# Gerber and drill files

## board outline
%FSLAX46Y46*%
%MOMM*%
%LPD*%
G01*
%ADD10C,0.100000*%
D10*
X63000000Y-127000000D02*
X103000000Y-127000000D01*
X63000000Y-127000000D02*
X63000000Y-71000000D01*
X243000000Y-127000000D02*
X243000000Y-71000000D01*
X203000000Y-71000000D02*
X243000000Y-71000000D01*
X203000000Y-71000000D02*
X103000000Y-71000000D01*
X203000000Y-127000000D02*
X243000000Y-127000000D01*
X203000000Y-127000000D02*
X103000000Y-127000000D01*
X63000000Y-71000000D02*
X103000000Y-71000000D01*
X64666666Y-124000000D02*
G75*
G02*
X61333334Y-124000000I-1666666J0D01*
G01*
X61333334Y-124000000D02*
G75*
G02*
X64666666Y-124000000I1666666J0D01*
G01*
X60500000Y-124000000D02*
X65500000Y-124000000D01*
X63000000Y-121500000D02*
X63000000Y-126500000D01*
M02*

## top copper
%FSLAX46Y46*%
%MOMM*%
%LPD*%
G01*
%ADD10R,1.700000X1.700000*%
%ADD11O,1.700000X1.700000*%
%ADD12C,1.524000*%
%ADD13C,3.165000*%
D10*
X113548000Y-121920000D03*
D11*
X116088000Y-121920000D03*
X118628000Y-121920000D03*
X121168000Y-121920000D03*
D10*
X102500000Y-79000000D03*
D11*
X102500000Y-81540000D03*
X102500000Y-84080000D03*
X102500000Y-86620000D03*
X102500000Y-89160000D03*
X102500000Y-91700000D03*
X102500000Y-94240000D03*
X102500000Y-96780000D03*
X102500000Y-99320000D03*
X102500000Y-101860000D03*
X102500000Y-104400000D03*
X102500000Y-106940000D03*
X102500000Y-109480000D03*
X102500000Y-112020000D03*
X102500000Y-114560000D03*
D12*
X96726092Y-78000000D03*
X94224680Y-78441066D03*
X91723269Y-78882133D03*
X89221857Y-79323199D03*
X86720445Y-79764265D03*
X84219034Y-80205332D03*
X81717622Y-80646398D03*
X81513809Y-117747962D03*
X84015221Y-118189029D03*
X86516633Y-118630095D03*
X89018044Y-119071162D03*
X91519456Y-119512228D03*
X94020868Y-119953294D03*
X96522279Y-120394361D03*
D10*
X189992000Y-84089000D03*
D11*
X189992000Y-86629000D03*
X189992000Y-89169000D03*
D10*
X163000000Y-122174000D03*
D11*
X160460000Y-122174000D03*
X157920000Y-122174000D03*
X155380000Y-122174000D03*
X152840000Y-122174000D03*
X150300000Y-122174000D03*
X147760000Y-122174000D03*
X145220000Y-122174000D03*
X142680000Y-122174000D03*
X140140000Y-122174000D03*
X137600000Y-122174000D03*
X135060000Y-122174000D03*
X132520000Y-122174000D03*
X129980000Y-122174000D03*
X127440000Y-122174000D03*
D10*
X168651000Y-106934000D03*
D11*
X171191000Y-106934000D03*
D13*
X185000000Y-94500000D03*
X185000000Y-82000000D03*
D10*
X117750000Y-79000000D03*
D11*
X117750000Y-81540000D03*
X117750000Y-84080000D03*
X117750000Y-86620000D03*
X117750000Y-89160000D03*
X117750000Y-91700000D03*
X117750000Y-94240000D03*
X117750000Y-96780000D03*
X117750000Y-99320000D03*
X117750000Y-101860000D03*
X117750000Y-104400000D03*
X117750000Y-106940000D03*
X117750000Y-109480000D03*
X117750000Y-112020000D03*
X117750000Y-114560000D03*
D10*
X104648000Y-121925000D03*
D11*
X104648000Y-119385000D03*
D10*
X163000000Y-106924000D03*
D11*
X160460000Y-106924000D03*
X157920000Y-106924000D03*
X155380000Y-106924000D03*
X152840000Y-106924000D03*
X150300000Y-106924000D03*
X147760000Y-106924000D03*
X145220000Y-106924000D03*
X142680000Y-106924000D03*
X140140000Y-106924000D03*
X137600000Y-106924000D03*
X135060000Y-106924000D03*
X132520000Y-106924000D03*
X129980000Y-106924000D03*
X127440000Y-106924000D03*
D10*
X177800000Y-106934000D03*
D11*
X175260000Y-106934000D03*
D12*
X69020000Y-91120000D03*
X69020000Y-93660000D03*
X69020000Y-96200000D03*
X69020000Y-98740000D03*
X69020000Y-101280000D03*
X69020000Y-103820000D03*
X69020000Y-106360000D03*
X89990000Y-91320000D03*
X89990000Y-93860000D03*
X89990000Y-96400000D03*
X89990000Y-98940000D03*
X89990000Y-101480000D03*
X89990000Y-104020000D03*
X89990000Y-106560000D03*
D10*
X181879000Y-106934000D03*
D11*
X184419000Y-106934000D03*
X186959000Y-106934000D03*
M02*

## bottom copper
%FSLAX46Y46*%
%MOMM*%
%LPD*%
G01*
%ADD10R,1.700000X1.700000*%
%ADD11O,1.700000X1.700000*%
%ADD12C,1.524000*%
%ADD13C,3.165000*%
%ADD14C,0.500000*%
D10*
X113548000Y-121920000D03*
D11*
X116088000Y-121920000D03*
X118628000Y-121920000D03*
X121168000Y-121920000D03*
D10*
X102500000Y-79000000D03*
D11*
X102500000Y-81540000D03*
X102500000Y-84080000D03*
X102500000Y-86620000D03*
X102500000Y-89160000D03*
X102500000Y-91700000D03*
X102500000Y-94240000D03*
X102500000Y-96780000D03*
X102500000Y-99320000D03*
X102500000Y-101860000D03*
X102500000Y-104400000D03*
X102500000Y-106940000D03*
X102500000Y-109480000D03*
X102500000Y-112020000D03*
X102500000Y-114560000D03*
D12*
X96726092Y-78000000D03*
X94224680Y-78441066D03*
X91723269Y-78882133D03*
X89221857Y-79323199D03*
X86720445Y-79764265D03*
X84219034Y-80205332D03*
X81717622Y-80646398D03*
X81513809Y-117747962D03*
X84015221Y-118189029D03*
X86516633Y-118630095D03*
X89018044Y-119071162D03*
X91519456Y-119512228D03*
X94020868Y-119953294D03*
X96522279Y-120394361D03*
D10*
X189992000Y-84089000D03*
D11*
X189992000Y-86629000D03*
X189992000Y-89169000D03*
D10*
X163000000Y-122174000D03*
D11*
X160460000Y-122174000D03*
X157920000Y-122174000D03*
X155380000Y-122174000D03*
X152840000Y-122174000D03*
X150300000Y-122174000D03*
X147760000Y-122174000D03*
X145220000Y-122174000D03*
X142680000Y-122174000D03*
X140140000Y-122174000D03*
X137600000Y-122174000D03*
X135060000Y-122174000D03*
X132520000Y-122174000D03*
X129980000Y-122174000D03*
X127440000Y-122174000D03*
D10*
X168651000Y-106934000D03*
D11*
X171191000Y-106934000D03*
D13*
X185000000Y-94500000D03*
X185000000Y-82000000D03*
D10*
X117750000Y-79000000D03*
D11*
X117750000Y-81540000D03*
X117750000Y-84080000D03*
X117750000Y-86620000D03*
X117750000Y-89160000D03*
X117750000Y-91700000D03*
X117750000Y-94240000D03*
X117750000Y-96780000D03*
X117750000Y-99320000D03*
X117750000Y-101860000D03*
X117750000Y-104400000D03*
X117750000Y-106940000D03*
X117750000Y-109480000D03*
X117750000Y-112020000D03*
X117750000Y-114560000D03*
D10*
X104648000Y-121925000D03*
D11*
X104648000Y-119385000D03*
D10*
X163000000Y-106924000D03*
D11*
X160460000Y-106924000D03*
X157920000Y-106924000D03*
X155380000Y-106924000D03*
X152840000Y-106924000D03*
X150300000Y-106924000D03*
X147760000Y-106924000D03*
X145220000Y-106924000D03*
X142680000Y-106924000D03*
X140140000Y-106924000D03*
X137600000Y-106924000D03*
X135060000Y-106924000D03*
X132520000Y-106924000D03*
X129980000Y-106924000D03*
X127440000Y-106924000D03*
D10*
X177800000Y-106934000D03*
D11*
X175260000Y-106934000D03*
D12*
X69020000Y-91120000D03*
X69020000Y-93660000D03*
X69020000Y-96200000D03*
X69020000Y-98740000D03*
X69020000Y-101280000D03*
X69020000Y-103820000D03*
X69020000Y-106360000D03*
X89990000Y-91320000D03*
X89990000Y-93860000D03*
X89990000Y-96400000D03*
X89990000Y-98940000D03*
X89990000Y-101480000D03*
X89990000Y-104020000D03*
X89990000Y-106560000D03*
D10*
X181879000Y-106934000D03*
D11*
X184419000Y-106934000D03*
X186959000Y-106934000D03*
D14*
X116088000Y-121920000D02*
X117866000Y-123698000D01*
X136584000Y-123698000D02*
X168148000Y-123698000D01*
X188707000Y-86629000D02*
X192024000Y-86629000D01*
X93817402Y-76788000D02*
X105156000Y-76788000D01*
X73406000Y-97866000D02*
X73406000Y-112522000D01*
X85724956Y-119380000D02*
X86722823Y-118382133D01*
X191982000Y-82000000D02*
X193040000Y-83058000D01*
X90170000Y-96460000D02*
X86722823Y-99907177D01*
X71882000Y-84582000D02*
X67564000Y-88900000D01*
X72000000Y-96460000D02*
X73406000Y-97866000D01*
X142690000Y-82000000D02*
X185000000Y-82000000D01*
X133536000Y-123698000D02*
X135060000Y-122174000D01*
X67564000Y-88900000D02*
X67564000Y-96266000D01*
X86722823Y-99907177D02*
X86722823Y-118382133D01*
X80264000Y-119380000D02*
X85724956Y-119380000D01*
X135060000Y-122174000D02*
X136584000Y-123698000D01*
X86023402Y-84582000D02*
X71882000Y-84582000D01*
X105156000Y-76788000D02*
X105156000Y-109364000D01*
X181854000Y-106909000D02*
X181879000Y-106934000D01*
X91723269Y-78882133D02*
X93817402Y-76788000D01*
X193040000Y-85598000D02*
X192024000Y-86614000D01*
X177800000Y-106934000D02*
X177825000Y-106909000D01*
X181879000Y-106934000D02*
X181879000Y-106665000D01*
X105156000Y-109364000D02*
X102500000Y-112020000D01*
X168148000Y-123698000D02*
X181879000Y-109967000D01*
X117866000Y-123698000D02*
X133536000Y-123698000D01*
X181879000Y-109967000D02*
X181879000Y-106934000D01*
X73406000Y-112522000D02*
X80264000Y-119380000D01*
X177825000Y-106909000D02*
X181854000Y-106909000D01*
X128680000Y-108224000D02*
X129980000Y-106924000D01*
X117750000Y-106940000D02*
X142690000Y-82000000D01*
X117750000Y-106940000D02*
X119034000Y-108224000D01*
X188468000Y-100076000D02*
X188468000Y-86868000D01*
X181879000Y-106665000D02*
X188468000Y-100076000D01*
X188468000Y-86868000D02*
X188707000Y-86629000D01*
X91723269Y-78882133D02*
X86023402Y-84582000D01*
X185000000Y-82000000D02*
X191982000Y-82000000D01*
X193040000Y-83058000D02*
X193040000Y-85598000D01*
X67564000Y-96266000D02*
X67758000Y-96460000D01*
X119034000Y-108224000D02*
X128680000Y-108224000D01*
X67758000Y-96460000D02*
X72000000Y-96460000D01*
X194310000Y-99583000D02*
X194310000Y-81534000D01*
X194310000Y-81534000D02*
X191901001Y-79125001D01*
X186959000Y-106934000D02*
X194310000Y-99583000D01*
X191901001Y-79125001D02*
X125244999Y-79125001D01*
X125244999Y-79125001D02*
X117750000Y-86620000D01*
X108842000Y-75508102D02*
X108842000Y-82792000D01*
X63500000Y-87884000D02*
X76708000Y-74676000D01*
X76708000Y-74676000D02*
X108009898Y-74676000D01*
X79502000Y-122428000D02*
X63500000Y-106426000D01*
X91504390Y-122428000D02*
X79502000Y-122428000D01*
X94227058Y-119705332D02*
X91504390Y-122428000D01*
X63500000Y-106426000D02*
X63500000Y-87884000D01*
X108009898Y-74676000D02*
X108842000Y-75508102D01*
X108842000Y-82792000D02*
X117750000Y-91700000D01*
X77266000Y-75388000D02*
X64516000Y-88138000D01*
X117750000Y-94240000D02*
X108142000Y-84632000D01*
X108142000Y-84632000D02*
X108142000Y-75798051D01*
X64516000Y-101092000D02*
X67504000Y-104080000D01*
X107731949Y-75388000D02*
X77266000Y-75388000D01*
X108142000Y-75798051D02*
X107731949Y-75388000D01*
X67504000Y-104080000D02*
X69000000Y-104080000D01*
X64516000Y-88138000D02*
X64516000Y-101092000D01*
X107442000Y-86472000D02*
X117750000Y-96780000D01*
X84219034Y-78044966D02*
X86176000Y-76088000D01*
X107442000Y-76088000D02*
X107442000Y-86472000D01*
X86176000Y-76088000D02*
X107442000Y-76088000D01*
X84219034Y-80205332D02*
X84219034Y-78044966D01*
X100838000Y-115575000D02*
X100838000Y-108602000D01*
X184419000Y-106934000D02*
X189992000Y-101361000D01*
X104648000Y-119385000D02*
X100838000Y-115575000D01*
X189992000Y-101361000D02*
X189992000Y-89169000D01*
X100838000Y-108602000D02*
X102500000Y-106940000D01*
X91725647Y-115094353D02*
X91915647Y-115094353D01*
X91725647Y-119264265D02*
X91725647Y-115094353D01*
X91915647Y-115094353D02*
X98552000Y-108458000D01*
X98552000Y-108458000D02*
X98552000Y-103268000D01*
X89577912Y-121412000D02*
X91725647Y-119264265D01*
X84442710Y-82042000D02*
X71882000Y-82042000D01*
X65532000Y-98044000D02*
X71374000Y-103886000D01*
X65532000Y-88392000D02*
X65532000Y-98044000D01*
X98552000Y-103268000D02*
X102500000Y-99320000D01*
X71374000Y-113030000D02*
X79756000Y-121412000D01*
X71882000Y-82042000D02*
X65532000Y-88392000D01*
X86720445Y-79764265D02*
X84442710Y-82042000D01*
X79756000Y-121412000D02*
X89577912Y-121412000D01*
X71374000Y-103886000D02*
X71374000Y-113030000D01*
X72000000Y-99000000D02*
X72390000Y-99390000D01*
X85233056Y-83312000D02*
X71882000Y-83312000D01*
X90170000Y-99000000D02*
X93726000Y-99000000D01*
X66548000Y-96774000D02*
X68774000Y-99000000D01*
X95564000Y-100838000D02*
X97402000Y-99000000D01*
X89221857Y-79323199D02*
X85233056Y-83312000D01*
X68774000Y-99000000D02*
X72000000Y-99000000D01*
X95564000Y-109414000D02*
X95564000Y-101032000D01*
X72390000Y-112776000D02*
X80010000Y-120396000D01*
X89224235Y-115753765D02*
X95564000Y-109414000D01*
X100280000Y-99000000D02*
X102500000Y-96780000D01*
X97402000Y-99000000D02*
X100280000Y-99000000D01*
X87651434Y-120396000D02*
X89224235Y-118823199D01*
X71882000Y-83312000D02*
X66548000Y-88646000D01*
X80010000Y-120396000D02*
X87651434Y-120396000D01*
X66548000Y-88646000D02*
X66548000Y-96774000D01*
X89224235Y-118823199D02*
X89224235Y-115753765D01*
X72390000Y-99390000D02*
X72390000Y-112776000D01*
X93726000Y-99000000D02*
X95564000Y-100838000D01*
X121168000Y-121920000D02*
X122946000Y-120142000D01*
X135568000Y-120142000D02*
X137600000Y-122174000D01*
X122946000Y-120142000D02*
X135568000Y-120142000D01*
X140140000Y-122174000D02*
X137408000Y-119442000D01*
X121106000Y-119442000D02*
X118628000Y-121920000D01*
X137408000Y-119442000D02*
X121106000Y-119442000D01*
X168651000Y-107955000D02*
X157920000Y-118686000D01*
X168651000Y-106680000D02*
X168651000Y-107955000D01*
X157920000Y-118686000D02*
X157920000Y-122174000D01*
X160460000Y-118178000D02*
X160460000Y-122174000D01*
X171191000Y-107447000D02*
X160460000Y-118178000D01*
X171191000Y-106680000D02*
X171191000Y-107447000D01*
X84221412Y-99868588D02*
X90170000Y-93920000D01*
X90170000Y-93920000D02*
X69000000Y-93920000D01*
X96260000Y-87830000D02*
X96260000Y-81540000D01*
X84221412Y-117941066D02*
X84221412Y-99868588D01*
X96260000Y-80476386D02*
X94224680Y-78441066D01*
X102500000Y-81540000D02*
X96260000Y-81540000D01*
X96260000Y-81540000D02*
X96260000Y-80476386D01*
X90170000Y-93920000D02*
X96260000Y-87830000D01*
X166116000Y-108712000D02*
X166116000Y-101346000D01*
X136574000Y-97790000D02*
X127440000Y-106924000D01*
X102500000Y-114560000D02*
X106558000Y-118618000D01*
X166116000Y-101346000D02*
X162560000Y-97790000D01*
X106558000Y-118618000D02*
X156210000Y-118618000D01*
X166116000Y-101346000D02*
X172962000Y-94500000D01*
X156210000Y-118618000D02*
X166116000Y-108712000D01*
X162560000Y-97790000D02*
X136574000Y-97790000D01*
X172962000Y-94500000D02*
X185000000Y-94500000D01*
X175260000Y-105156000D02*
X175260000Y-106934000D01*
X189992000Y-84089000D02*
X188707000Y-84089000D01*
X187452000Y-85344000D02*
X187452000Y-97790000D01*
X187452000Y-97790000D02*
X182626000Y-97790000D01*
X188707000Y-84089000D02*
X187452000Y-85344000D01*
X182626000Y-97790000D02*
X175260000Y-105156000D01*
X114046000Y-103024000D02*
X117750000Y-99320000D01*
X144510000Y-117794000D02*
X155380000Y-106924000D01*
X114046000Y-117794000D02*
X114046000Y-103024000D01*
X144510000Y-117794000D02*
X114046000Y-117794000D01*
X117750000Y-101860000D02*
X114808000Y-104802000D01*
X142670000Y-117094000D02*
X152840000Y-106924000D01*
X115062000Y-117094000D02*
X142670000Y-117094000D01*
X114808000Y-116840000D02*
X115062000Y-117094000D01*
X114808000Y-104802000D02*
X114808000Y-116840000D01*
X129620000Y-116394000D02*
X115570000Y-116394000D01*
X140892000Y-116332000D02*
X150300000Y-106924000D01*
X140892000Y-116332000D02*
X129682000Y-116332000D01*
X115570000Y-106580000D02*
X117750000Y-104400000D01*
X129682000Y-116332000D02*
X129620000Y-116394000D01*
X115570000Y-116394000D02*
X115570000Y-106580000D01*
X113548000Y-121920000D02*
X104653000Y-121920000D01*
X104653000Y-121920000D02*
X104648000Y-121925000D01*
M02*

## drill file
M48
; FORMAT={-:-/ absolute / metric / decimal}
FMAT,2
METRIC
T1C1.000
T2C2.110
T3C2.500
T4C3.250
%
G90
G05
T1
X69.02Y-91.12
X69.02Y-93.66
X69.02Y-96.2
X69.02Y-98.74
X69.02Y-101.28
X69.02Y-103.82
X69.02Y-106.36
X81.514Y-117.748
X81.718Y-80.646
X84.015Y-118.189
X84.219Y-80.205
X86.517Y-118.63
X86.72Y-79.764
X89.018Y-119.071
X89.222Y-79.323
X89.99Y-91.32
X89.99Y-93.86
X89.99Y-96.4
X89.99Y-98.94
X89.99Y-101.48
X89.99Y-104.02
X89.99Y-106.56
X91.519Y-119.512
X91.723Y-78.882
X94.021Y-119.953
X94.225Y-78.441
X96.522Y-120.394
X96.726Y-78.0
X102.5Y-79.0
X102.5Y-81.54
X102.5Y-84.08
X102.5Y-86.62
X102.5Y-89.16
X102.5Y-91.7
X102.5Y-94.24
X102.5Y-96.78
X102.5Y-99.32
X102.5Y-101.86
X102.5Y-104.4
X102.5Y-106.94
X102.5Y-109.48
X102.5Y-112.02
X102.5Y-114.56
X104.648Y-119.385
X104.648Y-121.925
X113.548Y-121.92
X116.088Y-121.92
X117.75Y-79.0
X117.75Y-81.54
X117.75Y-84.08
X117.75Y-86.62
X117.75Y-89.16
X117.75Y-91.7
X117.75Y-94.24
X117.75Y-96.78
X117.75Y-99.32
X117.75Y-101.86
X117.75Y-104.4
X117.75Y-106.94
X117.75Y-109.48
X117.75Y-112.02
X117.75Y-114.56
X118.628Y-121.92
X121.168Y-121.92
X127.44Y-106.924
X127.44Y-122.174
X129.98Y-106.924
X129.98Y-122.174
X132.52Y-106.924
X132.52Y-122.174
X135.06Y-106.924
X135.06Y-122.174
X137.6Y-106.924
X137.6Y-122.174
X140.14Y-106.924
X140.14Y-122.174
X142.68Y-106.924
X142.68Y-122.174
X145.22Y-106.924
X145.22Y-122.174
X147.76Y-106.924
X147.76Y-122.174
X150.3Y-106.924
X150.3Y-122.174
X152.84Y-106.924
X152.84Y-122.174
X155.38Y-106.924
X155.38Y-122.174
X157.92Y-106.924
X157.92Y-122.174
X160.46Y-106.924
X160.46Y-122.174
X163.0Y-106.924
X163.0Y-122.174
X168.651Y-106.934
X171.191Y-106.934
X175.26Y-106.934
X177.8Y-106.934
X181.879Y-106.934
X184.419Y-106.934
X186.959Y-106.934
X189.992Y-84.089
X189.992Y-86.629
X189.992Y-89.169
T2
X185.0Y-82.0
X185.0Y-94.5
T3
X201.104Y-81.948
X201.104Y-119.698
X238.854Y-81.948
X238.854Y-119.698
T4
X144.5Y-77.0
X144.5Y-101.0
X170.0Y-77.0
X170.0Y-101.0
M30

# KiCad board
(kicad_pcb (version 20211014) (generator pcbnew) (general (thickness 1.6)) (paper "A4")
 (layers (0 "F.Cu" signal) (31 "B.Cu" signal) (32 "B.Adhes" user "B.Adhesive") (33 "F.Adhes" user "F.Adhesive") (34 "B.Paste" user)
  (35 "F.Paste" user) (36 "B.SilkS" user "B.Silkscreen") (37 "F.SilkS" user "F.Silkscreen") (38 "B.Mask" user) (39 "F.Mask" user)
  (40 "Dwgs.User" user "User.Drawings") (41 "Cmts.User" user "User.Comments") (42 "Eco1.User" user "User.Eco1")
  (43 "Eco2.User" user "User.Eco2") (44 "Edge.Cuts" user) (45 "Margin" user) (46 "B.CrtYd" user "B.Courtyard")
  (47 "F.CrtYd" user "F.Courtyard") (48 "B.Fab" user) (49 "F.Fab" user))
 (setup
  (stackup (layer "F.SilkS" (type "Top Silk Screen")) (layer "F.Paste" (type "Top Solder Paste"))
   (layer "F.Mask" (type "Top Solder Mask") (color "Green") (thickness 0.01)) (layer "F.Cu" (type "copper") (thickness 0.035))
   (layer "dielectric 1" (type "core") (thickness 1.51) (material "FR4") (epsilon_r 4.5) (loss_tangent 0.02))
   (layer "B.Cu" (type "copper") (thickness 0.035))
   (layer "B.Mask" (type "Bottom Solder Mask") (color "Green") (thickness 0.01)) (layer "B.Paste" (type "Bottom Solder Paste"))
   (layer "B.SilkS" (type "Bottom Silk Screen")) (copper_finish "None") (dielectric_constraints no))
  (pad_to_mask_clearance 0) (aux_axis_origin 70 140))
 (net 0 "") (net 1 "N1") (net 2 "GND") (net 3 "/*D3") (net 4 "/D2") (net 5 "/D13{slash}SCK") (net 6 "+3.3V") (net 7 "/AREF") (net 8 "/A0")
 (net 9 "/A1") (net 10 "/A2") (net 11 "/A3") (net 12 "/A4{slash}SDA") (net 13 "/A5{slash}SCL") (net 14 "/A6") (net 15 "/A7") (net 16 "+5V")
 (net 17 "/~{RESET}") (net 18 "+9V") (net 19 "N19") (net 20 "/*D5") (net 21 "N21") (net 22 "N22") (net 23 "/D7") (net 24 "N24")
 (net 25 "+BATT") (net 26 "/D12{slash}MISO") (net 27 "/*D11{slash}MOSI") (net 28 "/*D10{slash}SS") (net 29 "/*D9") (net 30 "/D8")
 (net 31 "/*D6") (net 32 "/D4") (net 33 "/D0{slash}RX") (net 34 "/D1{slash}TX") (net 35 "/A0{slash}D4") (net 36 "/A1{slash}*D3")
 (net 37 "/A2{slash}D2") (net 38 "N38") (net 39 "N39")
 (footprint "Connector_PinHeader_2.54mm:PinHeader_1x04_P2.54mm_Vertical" (layer "F.Cu") (at 113.548 121.92 90)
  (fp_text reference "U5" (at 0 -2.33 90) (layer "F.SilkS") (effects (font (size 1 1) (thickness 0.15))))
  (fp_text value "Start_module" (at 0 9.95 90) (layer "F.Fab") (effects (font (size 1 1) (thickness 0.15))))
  (pad "1" thru_hole rect (at 0 0 90) (size 1.7 1.7) (drill 1) (layers *.Cu *.Mask) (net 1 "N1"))
  (pad "2" thru_hole oval (at 0 2.54 90) (size 1.7 1.7) (drill 1) (layers *.Cu *.Mask) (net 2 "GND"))
  (pad "3" thru_hole oval (at 0 5.08 90) (size 1.7 1.7) (drill 1) (layers *.Cu *.Mask) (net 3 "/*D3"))
  (pad "4" thru_hole oval (at 0 7.62 90) (size 1.7 1.7) (drill 1) (layers *.Cu *.Mask) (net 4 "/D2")))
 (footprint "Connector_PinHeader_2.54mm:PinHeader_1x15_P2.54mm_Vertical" (layer "F.Cu") (at 102.5 79)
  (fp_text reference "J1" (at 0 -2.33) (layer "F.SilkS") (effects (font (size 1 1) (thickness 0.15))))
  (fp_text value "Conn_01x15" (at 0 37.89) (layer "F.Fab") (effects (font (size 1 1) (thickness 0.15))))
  (pad "1" thru_hole rect (at 0 0) (size 1.7 1.7) (drill 1) (layers *.Cu *.Mask) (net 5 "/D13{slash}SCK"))
  (pad "2" thru_hole oval (at 0 2.54) (size 1.7 1.7) (drill 1) (layers *.Cu *.Mask) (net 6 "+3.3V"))
  (pad "3" thru_hole oval (at 0 5.08) (size 1.7 1.7) (drill 1) (layers *.Cu *.Mask) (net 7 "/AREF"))
  (pad "4" thru_hole oval (at 0 7.62) (size 1.7 1.7) (drill 1) (layers *.Cu *.Mask) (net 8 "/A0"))
  (pad "5" thru_hole oval (at 0 10.16) (size 1.7 1.7) (drill 1) (layers *.Cu *.Mask) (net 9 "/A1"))
  (pad "6" thru_hole oval (at 0 12.7) (size 1.7 1.7) (drill 1) (layers *.Cu *.Mask) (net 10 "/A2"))
  (pad "7" thru_hole oval (at 0 15.24) (size 1.7 1.7) (drill 1) (layers *.Cu *.Mask) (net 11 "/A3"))
  (pad "8" thru_hole oval (at 0 17.78) (size 1.7 1.7) (drill 1) (layers *.Cu *.Mask) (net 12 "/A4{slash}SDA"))
  (pad "9" thru_hole oval (at 0 20.32) (size 1.7 1.7) (drill 1) (layers *.Cu *.Mask) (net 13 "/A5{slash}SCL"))
  (pad "10" thru_hole oval (at 0 22.86) (size 1.7 1.7) (drill 1) (layers *.Cu *.Mask) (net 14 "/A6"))
  (pad "11" thru_hole oval (at 0 25.4) (size 1.7 1.7) (drill 1) (layers *.Cu *.Mask) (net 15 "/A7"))
  (pad "12" thru_hole oval (at 0 27.94) (size 1.7 1.7) (drill 1) (layers *.Cu *.Mask) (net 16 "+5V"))
  (pad "13" thru_hole oval (at 0 30.48) (size 1.7 1.7) (drill 1) (layers *.Cu *.Mask) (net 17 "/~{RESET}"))
  (pad "14" thru_hole oval (at 0 33.02) (size 1.7 1.7) (drill 1) (layers *.Cu *.Mask) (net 2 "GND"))
  (pad "15" thru_hole oval (at 0 35.56) (size 1.7 1.7) (drill 1) (layers *.Cu *.Mask) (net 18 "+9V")))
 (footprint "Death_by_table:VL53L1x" (layer "F.Cu") (at 96.726092 78 -170)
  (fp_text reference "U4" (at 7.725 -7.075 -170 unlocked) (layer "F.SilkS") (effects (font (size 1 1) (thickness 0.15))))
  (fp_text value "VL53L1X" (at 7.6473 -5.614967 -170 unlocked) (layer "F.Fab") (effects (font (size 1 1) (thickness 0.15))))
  (pad "1" thru_hole circle (at 0 0 190) (size 1.524 1.524) (drill 1) (layers *.Cu *.Mask) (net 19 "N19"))
  (pad "2" thru_hole circle (at 2.54 0 190) (size 1.524 1.524) (drill 1) (layers *.Cu *.Mask) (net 6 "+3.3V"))
  (pad "3" thru_hole circle (at 5.08 0 190) (size 1.524 1.524) (drill 1) (layers *.Cu *.Mask) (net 2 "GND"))
  (pad "4" thru_hole circle (at 7.62 0 190) (size 1.524 1.524) (drill 1) (layers *.Cu *.Mask) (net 12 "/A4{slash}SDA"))
  (pad "5" thru_hole circle (at 10.16 0 190) (size 1.524 1.524) (drill 1) (layers *.Cu *.Mask) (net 13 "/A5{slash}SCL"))
  (pad "6" thru_hole circle (at 12.7 0 190) (size 1.524 1.524) (drill 1) (layers *.Cu *.Mask) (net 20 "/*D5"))
  (pad "7" thru_hole circle (at 15.24 0 190) (size 1.524 1.524) (drill 1) (layers *.Cu *.Mask) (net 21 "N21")))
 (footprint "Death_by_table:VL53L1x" (layer "F.Cu") (at 81.72 117.5 -10)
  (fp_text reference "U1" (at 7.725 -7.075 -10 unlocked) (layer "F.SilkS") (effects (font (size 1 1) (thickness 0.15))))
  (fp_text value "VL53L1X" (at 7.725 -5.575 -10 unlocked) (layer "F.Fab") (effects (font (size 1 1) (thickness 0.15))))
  (pad "1" thru_hole circle (at -0.16 0.28 350) (size 1.524 1.524) (drill 1) (layers *.Cu *.Mask) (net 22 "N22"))
  (pad "2" thru_hole circle (at 2.38 0.28 350) (size 1.524 1.524) (drill 1) (layers *.Cu *.Mask) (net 6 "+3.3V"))
  (pad "3" thru_hole circle (at 4.92 0.28 350) (size 1.524 1.524) (drill 1) (layers *.Cu *.Mask) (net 2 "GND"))
  (pad "4" thru_hole circle (at 7.46 0.28 350) (size 1.524 1.524) (drill 1) (layers *.Cu *.Mask) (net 12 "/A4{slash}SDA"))
  (pad "5" thru_hole circle (at 10 0.28 350) (size 1.524 1.524) (drill 1) (layers *.Cu *.Mask) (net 13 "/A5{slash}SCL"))
  (pad "6" thru_hole circle (at 12.54 0.28 350) (size 1.524 1.524) (drill 1) (layers *.Cu *.Mask) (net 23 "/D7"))
  (pad "7" thru_hole circle (at 15.08 0.28 350) (size 1.524 1.524) (drill 1) (layers *.Cu *.Mask) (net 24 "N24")))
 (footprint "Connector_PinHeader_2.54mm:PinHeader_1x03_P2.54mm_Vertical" (layer "F.Cu") (at 189.992 84.089)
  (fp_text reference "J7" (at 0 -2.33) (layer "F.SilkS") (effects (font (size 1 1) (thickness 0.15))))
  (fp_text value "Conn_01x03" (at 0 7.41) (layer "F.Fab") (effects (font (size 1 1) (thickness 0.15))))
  (pad "1" thru_hole rect (at 0 0) (size 1.7 1.7) (drill 1) (layers *.Cu *.Mask) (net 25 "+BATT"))
  (pad "2" thru_hole oval (at 0 2.54) (size 1.7 1.7) (drill 1) (layers *.Cu *.Mask) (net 2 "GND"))
  (pad "3" thru_hole oval (at 0 5.08) (size 1.7 1.7) (drill 1) (layers *.Cu *.Mask) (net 16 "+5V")))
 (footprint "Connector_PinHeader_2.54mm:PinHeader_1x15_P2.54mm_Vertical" (layer "F.Cu") (at 163 122.174 -90)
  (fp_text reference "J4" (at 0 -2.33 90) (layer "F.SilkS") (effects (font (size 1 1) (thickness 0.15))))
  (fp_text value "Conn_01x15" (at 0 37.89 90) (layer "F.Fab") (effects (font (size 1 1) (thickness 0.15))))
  (pad "1" thru_hole rect (at 0 0 270) (size 1.7 1.7) (drill 1) (layers *.Cu *.Mask) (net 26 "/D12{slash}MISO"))
  (pad "2" thru_hole oval (at 0 2.54 270) (size 1.7 1.7) (drill 1) (layers *.Cu *.Mask) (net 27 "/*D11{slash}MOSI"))
  (pad "3" thru_hole oval (at 0 5.08 270) (size 1.7 1.7) (drill 1) (layers *.Cu *.Mask) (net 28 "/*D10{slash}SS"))
  (pad "4" thru_hole oval (at 0 7.62 270) (size 1.7 1.7) (drill 1) (layers *.Cu *.Mask) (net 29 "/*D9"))
  (pad "5" thru_hole oval (at 0 10.16 270) (size 1.7 1.7) (drill 1) (layers *.Cu *.Mask) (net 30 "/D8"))
  (pad "6" thru_hole oval (at 0 12.7 270) (size 1.7 1.7) (drill 1) (layers *.Cu *.Mask) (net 23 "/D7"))
  (pad "7" thru_hole oval (at 0 15.24 270) (size 1.7 1.7) (drill 1) (layers *.Cu *.Mask) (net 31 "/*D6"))
  (pad "8" thru_hole oval (at 0 17.78 270) (size 1.7 1.7) (drill 1) (layers *.Cu *.Mask) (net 20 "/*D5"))
  (pad "9" thru_hole oval (at 0 20.32 270) (size 1.7 1.7) (drill 1) (layers *.Cu *.Mask) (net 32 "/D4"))
  (pad "10" thru_hole oval (at 0 22.86 270) (size 1.7 1.7) (drill 1) (layers *.Cu *.Mask) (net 3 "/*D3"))
  (pad "11" thru_hole oval (at 0 25.4 270) (size 1.7 1.7) (drill 1) (layers *.Cu *.Mask) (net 4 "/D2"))
  (pad "12" thru_hole oval (at 0 27.94 270) (size 1.7 1.7) (drill 1) (layers *.Cu *.Mask) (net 2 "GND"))
  (pad "13" thru_hole oval (at 0 30.48 270) (size 1.7 1.7) (drill 1) (layers *.Cu *.Mask) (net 17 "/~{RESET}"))
  (pad "14" thru_hole oval (at 0 33.02 270) (size 1.7 1.7) (drill 1) (layers *.Cu *.Mask) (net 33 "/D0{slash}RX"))
  (pad "15" thru_hole oval (at 0 35.56 270) (size 1.7 1.7) (drill 1) (layers *.Cu *.Mask) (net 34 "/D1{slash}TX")))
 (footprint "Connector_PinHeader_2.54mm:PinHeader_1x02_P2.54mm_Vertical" (layer "F.Cu") (at 168.651 106.934 90)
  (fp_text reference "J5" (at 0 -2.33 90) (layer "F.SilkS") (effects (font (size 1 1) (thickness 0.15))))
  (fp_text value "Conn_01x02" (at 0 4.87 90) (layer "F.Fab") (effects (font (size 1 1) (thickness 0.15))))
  (pad "1" thru_hole rect (at 0 0 90) (size 1.7 1.7) (drill 1) (layers *.Cu *.Mask) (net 28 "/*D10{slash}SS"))
  (pad "2" thru_hole oval (at 0 2.54 90) (size 1.7 1.7) (drill 1) (layers *.Cu *.Mask) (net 27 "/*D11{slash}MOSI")))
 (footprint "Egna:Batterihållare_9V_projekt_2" (layer "F.Cu") (at 185 74 180)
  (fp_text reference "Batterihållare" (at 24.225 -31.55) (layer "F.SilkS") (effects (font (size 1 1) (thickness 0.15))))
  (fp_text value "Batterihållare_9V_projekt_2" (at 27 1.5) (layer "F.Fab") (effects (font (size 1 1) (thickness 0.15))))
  (pad "" np_thru_hole circle (at 15 -27 180) (size 2.3 2.3) (drill 3.25) (layers F&B.Cu *.Mask))
  (pad "" np_thru_hole circle (at 40.5 -3 180) (size 2.3 2.3) (drill 3.25) (layers F&B.Cu *.Mask))
  (pad "" np_thru_hole circle (at 15 -3 180) (size 2.3 2.3) (drill 3.25) (layers F&B.Cu *.Mask))
  (pad "" np_thru_hole circle (at 40.5 -27 180) (size 2.3 2.3) (drill 3.25) (layers F&B.Cu *.Mask))
  (pad "1" thru_hole circle (at 0 -20.5 180) (size 3.165 3.165) (drill 2.11) (layers *.Cu *.Mask) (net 18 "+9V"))
  (pad "2" thru_hole circle (at 0 -8 180) (size 3.165 3.165) (drill 2.11) (layers *.Cu *.Mask) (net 2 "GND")))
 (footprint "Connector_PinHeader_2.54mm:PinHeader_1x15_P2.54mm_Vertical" (layer "F.Cu") (at 117.75 79)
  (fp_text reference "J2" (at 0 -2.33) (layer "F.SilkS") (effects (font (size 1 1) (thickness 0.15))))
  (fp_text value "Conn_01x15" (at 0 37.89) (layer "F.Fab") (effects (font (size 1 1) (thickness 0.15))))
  (pad "1" thru_hole rect (at 0 0) (size 1.7 1.7) (drill 1) (layers *.Cu *.Mask) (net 26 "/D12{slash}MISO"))
  (pad "2" thru_hole oval (at 0 2.54) (size 1.7 1.7) (drill 1) (layers *.Cu *.Mask) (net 27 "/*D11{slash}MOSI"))
  (pad "3" thru_hole oval (at 0 5.08) (size 1.7 1.7) (drill 1) (layers *.Cu *.Mask) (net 28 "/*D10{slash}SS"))
  (pad "4" thru_hole oval (at 0 7.62) (size 1.7 1.7) (drill 1) (layers *.Cu *.Mask) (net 29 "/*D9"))
  (pad "5" thru_hole oval (at 0 10.16) (size 1.7 1.7) (drill 1) (layers *.Cu *.Mask) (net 30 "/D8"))
  (pad "6" thru_hole oval (at 0 12.7) (size 1.7 1.7) (drill 1) (layers *.Cu *.Mask) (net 23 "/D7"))
  (pad "7" thru_hole oval (at 0 15.24) (size 1.7 1.7) (drill 1) (layers *.Cu *.Mask) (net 31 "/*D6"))
  (pad "8" thru_hole oval (at 0 17.78) (size 1.7 1.7) (drill 1) (layers *.Cu *.Mask) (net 20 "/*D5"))
  (pad "9" thru_hole oval (at 0 20.32) (size 1.7 1.7) (drill 1) (layers *.Cu *.Mask) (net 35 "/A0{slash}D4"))
  (pad "10" thru_hole oval (at 0 22.86) (size 1.7 1.7) (drill 1) (layers *.Cu *.Mask) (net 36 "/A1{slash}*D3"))
  (pad "11" thru_hole oval (at 0 25.4) (size 1.7 1.7) (drill 1) (layers *.Cu *.Mask) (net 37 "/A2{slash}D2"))
  (pad "12" thru_hole oval (at 0 27.94) (size 1.7 1.7) (drill 1) (layers *.Cu *.Mask) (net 2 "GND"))
  (pad "13" thru_hole oval (at 0 30.48) (size 1.7 1.7) (drill 1) (layers *.Cu *.Mask) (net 17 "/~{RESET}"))
  (pad "14" thru_hole oval (at 0 33.02) (size 1.7 1.7) (drill 1) (layers *.Cu *.Mask) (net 33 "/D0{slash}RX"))
  (pad "15" thru_hole oval (at 0 35.56) (size 1.7 1.7) (drill 1) (layers *.Cu *.Mask) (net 34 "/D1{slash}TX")))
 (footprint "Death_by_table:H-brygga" (layer "F.Cu") (at 197.104 123.698)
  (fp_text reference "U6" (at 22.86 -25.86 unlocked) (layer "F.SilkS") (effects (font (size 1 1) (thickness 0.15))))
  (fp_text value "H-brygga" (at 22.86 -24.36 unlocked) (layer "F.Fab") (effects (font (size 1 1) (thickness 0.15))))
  (pad "" np_thru_hole circle (at 4 -4) (size 2.5 2.5) (drill 2.5) (layers F&B.Cu *.Mask))
  (pad "" np_thru_hole circle (at 41.75 -41.75) (size 2.5 2.5) (drill 2.5) (layers F&B.Cu *.Mask))
  (pad "" np_thru_hole circle (at 4 -41.75) (size 2.5 2.5) (drill 2.5) (layers F&B.Cu *.Mask))
  (pad "" np_thru_hole circle (at 41.75 -4) (size 2.5 2.5) (drill 2.5) (layers F&B.Cu *.Mask)))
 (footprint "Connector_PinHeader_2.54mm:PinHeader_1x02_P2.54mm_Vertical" (layer "F.Cu") (at 104.648 121.925 180)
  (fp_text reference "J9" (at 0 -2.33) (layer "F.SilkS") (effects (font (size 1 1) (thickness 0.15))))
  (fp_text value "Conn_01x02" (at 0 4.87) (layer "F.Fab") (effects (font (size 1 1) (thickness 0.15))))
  (pad "1" thru_hole rect (at 0 0 180) (size 1.7 1.7) (drill 1) (layers *.Cu *.Mask) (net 1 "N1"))
  (pad "2" thru_hole oval (at 0 2.54 180) (size 1.7 1.7) (drill 1) (layers *.Cu *.Mask) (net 16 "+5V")))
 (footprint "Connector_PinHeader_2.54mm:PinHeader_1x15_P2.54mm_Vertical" (layer "F.Cu") (at 163 106.924 -90)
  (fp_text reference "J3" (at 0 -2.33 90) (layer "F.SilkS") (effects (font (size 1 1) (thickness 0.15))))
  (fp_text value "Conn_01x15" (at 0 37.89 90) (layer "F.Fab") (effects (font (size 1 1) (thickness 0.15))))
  (pad "1" thru_hole rect (at 0 0 270) (size 1.7 1.7) (drill 1) (layers *.Cu *.Mask) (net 5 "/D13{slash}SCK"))
  (pad "2" thru_hole oval (at 0 2.54 270) (size 1.7 1.7) (drill 1) (layers *.Cu *.Mask) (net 6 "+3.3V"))
  (pad "3" thru_hole oval (at 0 5.08 270) (size 1.7 1.7) (drill 1) (layers *.Cu *.Mask) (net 7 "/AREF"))
  (pad "4" thru_hole oval (at 0 7.62 270) (size 1.7 1.7) (drill 1) (layers *.Cu *.Mask) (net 35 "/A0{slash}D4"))
  (pad "5" thru_hole oval (at 0 10.16 270) (size 1.7 1.7) (drill 1) (layers *.Cu *.Mask) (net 36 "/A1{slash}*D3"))
  (pad "6" thru_hole oval (at 0 12.7 270) (size 1.7 1.7) (drill 1) (layers *.Cu *.Mask) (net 37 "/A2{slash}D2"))
  (pad "7" thru_hole oval (at 0 15.24 270) (size 1.7 1.7) (drill 1) (layers *.Cu *.Mask) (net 11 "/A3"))
  (pad "8" thru_hole oval (at 0 17.78 270) (size 1.7 1.7) (drill 1) (layers *.Cu *.Mask) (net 12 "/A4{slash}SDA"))
  (pad "9" thru_hole oval (at 0 20.32 270) (size 1.7 1.7) (drill 1) (layers *.Cu *.Mask) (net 13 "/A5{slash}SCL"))
  (pad "10" thru_hole oval (at 0 22.86 270) (size 1.7 1.7) (drill 1) (layers *.Cu *.Mask) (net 14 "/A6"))
  (pad "11" thru_hole oval (at 0 25.4 270) (size 1.7 1.7) (drill 1) (layers *.Cu *.Mask) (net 15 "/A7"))
  (pad "12" thru_hole oval (at 0 27.94 270) (size 1.7 1.7) (drill 1) (layers *.Cu *.Mask) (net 16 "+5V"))
  (pad "13" thru_hole oval (at 0 30.48 270) (size 1.7 1.7) (drill 1) (layers *.Cu *.Mask) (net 17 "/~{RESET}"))
  (pad "14" thru_hole oval (at 0 33.02 270) (size 1.7 1.7) (drill 1) (layers *.Cu *.Mask) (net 2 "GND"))
  (pad "15" thru_hole oval (at 0 35.56 270) (size 1.7 1.7) (drill 1) (layers *.Cu *.Mask) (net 18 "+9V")))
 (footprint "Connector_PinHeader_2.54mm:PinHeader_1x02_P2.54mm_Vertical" (layer "F.Cu") (at 177.8 106.934 -90)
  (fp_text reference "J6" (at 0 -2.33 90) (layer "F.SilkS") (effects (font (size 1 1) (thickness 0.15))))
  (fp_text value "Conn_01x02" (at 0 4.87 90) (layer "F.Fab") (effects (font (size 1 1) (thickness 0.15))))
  (pad "1" thru_hole rect (at 0 0 270) (size 1.7 1.7) (drill 1) (layers *.Cu *.Mask) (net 2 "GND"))
  (pad "2" thru_hole oval (at 0 2.54 270) (size 1.7 1.7) (drill 1) (layers *.Cu *.Mask) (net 25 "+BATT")))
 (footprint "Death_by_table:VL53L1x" (layer "F.Cu") (at 69 91.38 -90)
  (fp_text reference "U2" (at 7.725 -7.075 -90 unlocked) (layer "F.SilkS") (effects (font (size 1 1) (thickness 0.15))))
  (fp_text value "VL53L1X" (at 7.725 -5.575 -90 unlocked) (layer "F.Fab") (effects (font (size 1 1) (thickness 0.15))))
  (pad "1" thru_hole circle (at -0.26 -0.02 270) (size 1.524 1.524) (drill 1) (layers *.Cu *.Mask) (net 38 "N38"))
  (pad "2" thru_hole circle (at 2.28 -0.02 270) (size 1.524 1.524) (drill 1) (layers *.Cu *.Mask) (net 6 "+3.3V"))
  (pad "3" thru_hole circle (at 4.82 -0.02 270) (size 1.524 1.524) (drill 1) (layers *.Cu *.Mask) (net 2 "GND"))
  (pad "4" thru_hole circle (at 7.36 -0.02 270) (size 1.524 1.524) (drill 1) (layers *.Cu *.Mask) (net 12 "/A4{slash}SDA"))
  (pad "5" thru_hole circle (at 9.9 -0.02 270) (size 1.524 1.524) (drill 1) (layers *.Cu *.Mask) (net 13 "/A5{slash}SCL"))
  (pad "6" thru_hole circle (at 12.44 -0.02 270) (size 1.524 1.524) (drill 1) (layers *.Cu *.Mask) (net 31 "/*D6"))
  (pad "7" thru_hole circle (at 14.98 -0.02 270) (size 1.524 1.524) (drill 1) (layers *.Cu *.Mask) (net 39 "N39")))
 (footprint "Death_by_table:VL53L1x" (layer "F.Cu") (at 90.17 91.38 -90)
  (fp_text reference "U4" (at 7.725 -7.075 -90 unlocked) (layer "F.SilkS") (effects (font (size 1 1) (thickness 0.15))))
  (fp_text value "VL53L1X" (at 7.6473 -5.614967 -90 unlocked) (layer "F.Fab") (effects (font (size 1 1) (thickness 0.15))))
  (pad "1" thru_hole circle (at -0.06 0.18 270) (size 1.524 1.524) (drill 1) (layers *.Cu *.Mask))
  (pad "2" thru_hole circle (at 2.48 0.18 270) (size 1.524 1.524) (drill 1) (layers *.Cu *.Mask) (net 6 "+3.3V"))
  (pad "3" thru_hole circle (at 5.02 0.18 270) (size 1.524 1.524) (drill 1) (layers *.Cu *.Mask) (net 2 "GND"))
  (pad "4" thru_hole circle (at 7.56 0.18 270) (size 1.524 1.524) (drill 1) (layers *.Cu *.Mask) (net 12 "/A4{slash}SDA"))
  (pad "5" thru_hole circle (at 10.1 0.18 270) (size 1.524 1.524) (drill 1) (layers *.Cu *.Mask) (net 13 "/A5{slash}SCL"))
  (pad "6" thru_hole circle (at 12.64 0.18 270) (size 1.524 1.524) (drill 1) (layers *.Cu *.Mask) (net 30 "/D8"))
  (pad "7" thru_hole circle (at 15.18 0.18 270) (size 1.524 1.524) (drill 1) (layers *.Cu *.Mask)))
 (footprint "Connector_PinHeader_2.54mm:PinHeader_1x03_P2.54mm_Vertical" (layer "F.Cu") (at 181.879 106.934 90)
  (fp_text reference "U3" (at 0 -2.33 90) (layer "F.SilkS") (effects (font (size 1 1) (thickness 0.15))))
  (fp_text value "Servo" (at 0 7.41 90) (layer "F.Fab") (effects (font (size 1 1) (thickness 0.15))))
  (pad "1" thru_hole rect (at 0 0 90) (size 1.7 1.7) (drill 1) (layers *.Cu *.Mask) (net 2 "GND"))
  (pad "2" thru_hole oval (at 0 2.54 90) (size 1.7 1.7) (drill 1) (layers *.Cu *.Mask) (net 16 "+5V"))
  (pad "3" thru_hole oval (at 0 5.08 90) (size 1.7 1.7) (drill 1) (layers *.Cu *.Mask) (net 29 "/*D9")))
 (gr_line (start 63 127) (end 103 127) (layer "Edge.Cuts") (width 0.1))
 (gr_line (start 63 127) (end 63 71) (layer "Edge.Cuts") (width 0.1))
 (gr_line (start 243 127) (end 243 71) (layer "Edge.Cuts") (width 0.1))
 (gr_line (start 203 71) (end 243 71) (layer "Edge.Cuts") (width 0.1))
 (gr_line (start 203 71) (end 103 71) (layer "Edge.Cuts") (width 0.1))
 (gr_line (start 203 127) (end 243 127) (layer "Edge.Cuts") (width 0.1))
 (gr_line (start 203 127) (end 103 127) (layer "Edge.Cuts") (width 0.1))
 (gr_line (start 63 71) (end 103 71) (layer "Edge.Cuts") (width 0.1))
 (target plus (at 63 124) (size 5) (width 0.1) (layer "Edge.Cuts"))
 (segment (start 116.088 121.92) (end 117.866 123.698) (width 0.5) (layer "B.Cu") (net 2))
 (segment (start 136.584 123.698) (end 168.148 123.698) (width 0.5) (layer "B.Cu") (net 2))
 (segment (start 188.707 86.629) (end 192.024 86.629) (width 0.5) (layer "B.Cu") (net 2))
 (segment (start 93.817402 76.788) (end 105.156 76.788) (width 0.5) (layer "B.Cu") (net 2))
 (segment (start 73.406 97.866) (end 73.406 112.522) (width 0.5) (layer "B.Cu") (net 2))
 (segment (start 85.724956 119.38) (end 86.722823 118.382133) (width 0.5) (layer "B.Cu") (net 2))
 (segment (start 191.982 82) (end 193.04 83.058) (width 0.5) (layer "B.Cu") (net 2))
 (segment (start 90.17 96.46) (end 86.722823 99.907177) (width 0.5) (layer "B.Cu") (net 2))
 (segment (start 71.882 84.582) (end 67.564 88.9) (width 0.5) (layer "B.Cu") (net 2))
 (segment (start 72 96.46) (end 73.406 97.866) (width 0.5) (layer "B.Cu") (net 2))
 (segment (start 142.69 82) (end 185 82) (width 0.5) (layer "B.Cu") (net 2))
 (segment (start 133.536 123.698) (end 135.06 122.174) (width 0.5) (layer "B.Cu") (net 2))
 (segment (start 67.564 88.9) (end 67.564 96.266) (width 0.5) (layer "B.Cu") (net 2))
 (segment (start 86.722823 99.907177) (end 86.722823 118.382133) (width 0.5) (layer "B.Cu") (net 2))
 (segment (start 80.264 119.38) (end 85.724956 119.38) (width 0.5) (layer "B.Cu") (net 2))
 (segment (start 135.06 122.174) (end 136.584 123.698) (width 0.5) (layer "B.Cu") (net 2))
 (segment (start 86.023402 84.582) (end 71.882 84.582) (width 0.5) (layer "B.Cu") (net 2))
 (segment (start 105.156 76.788) (end 105.156 109.364) (width 0.5) (layer "B.Cu") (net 2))
 (segment (start 181.854 106.909) (end 181.879 106.934) (width 0.5) (layer "B.Cu") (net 2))
 (segment (start 91.723269 78.882133) (end 93.817402 76.788) (width 0.5) (layer "B.Cu") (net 2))
 (segment (start 193.04 85.598) (end 192.024 86.614) (width 0.5) (layer "B.Cu") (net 2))
 (segment (start 177.8 106.934) (end 177.825 106.909) (width 0.5) (layer "B.Cu") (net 2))
 (segment (start 181.879 106.934) (end 181.879 106.665) (width 0.5) (layer "B.Cu") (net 2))
 (segment (start 105.156 109.364) (end 102.5 112.02) (width 0.5) (layer "B.Cu") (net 2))
 (segment (start 168.148 123.698) (end 181.879 109.967) (width 0.5) (layer "B.Cu") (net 2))
 (segment (start 117.866 123.698) (end 133.536 123.698) (width 0.5) (layer "B.Cu") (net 2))
 (segment (start 181.879 109.967) (end 181.879 106.934) (width 0.5) (layer "B.Cu") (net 2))
 (segment (start 73.406 112.522) (end 80.264 119.38) (width 0.5) (layer "B.Cu") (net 2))
 (segment (start 177.825 106.909) (end 181.854 106.909) (width 0.5) (layer "B.Cu") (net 2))
 (segment (start 128.68 108.224) (end 129.98 106.924) (width 0.5) (layer "B.Cu") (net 2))
 (segment (start 117.75 106.94) (end 142.69 82) (width 0.5) (layer "B.Cu") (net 2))
 (segment (start 117.75 106.94) (end 119.034 108.224) (width 0.5) (layer "B.Cu") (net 2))
 (segment (start 188.468 100.076) (end 188.468 86.868) (width 0.5) (layer "B.Cu") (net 2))
 (segment (start 181.879 106.665) (end 188.468 100.076) (width 0.5) (layer "B.Cu") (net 2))
 (segment (start 188.468 86.868) (end 188.707 86.629) (width 0.5) (layer "B.Cu") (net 2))
 (segment (start 91.723269 78.882133) (end 86.023402 84.582) (width 0.5) (layer "B.Cu") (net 2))
 (segment (start 185 82) (end 191.982 82) (width 0.5) (layer "B.Cu") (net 2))
 (segment (start 193.04 83.058) (end 193.04 85.598) (width 0.5) (layer "B.Cu") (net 2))
 (segment (start 67.564 96.266) (end 67.758 96.46) (width 0.5) (layer "B.Cu") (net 2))
 (segment (start 119.034 108.224) (end 128.68 108.224) (width 0.5) (layer "B.Cu") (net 2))
 (segment (start 67.758 96.46) (end 72 96.46) (width 0.5) (layer "B.Cu") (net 2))
 (segment (start 194.31 99.583) (end 194.31 81.534) (width 0.5) (layer "B.Cu") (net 29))
 (segment (start 194.31 81.534) (end 191.901001 79.125001) (width 0.5) (layer "B.Cu") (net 29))
 (segment (start 186.959 106.934) (end 194.31 99.583) (width 0.5) (layer "B.Cu") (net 29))
 (segment (start 191.901001 79.125001) (end 125.244999 79.125001) (width 0.5) (layer "B.Cu") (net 29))
 (segment (start 125.244999 79.125001) (end 117.75 86.62) (width 0.5) (layer "B.Cu") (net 29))
 (segment (start 108.842 75.508102) (end 108.842 82.792) (width 0.5) (layer "B.Cu") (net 23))
 (segment (start 63.5 87.884) (end 76.708 74.676) (width 0.5) (layer "B.Cu") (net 23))
 (segment (start 76.708 74.676) (end 108.009898 74.676) (width 0.5) (layer "B.Cu") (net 23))
 (segment (start 79.502 122.428) (end 63.5 106.426) (width 0.5) (layer "B.Cu") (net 23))
 (segment (start 91.50439 122.428) (end 79.502 122.428) (width 0.5) (layer "B.Cu") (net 23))
 (segment (start 94.227058 119.705332) (end 91.50439 122.428) (width 0.5) (layer "B.Cu") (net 23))
 (segment (start 63.5 106.426) (end 63.5 87.884) (width 0.5) (layer "B.Cu") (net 23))
 (segment (start 108.009898 74.676) (end 108.842 75.508102) (width 0.5) (layer "B.Cu") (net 23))
 (segment (start 108.842 82.792) (end 117.75 91.7) (width 0.5) (layer "B.Cu") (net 23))
 (segment (start 77.266 75.388) (end 64.516 88.138) (width 0.5) (layer "B.Cu") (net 31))
 (segment (start 117.75 94.24) (end 108.142 84.632) (width 0.5) (layer "B.Cu") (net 31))
 (segment (start 108.142 84.632) (end 108.142 75.798051) (width 0.5) (layer "B.Cu") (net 31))
 (segment (start 64.516 101.092) (end 67.504 104.08) (width 0.5) (layer "B.Cu") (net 31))
 (segment (start 107.731949 75.388) (end 77.266 75.388) (width 0.5) (layer "B.Cu") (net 31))
 (segment (start 108.142 75.798051) (end 107.731949 75.388) (width 0.5) (layer "B.Cu") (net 31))
 (segment (start 67.504 104.08) (end 69 104.08) (width 0.5) (layer "B.Cu") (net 31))
 (segment (start 64.516 88.138) (end 64.516 101.092) (width 0.5) (layer "B.Cu") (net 31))
 (segment (start 107.442 86.472) (end 117.75 96.78) (width 0.5) (layer "B.Cu") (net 20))
 (segment (start 84.219034 78.044966) (end 86.176 76.088) (width 0.5) (layer "B.Cu") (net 20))
 (segment (start 107.442 76.088) (end 107.442 86.472) (width 0.5) (layer "B.Cu") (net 20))
 (segment (start 86.176 76.088) (end 107.442 76.088) (width 0.5) (layer "B.Cu") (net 20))
 (segment (start 84.219034 80.205332) (end 84.219034 78.044966) (width 0.5) (layer "B.Cu") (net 20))
 (segment (start 100.838 115.575) (end 100.838 108.602) (width 0.5) (layer "B.Cu") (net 16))
 (segment (start 184.419 106.934) (end 189.992 101.361) (width 0.5) (layer "B.Cu") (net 16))
 (segment (start 104.648 119.385) (end 100.838 115.575) (width 0.5) (layer "B.Cu") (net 16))
 (segment (start 189.992 101.361) (end 189.992 89.169) (width 0.5) (layer "B.Cu") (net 16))
 (segment (start 100.838 108.602) (end 102.5 106.94) (width 0.5) (layer "B.Cu") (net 16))
 (segment (start 91.725647 115.094353) (end 91.915647 115.094353) (width 0.5) (layer "B.Cu") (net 13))
 (segment (start 91.725647 119.264265) (end 91.725647 115.094353) (width 0.5) (layer "B.Cu") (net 13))
 (segment (start 91.915647 115.094353) (end 98.552 108.458) (width 0.5) (layer "B.Cu") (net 13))
 (segment (start 98.552 108.458) (end 98.552 103.268) (width 0.5) (layer "B.Cu") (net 13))
 (segment (start 89.577912 121.412) (end 91.725647 119.264265) (width 0.5) (layer "B.Cu") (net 13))
 (segment (start 84.44271 82.042) (end 71.882 82.042) (width 0.5) (layer "B.Cu") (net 13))
 (segment (start 65.532 98.044) (end 71.374 103.886) (width 0.5) (layer "B.Cu") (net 13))
 (segment (start 65.532 88.392) (end 65.532 98.044) (width 0.5) (layer "B.Cu") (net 13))
 (segment (start 98.552 103.268) (end 102.5 99.32) (width 0.5) (layer "B.Cu") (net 13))
 (segment (start 71.374 113.03) (end 79.756 121.412) (width 0.5) (layer "B.Cu") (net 13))
 (segment (start 71.882 82.042) (end 65.532 88.392) (width 0.5) (layer "B.Cu") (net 13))
 (segment (start 86.720445 79.764265) (end 84.44271 82.042) (width 0.5) (layer "B.Cu") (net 13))
 (segment (start 79.756 121.412) (end 89.577912 121.412) (width 0.5) (layer "B.Cu") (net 13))
 (segment (start 71.374 103.886) (end 71.374 113.03) (width 0.5) (layer "B.Cu") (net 13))
 (segment (start 72 99) (end 72.39 99.39) (width 0.5) (layer "B.Cu") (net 12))
 (segment (start 85.233056 83.312) (end 71.882 83.312) (width 0.5) (layer "B.Cu") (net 12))
 (segment (start 90.17 99) (end 93.726 99) (width 0.5) (layer "B.Cu") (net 12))
 (segment (start 66.548 96.774) (end 68.774 99) (width 0.5) (layer "B.Cu") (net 12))
 (segment (start 95.564 100.838) (end 97.402 99) (width 0.5) (layer "B.Cu") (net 12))
 (segment (start 89.221857 79.323199) (end 85.233056 83.312) (width 0.5) (layer "B.Cu") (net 12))
 (segment (start 68.774 99) (end 72 99) (width 0.5) (layer "B.Cu") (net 12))
 (segment (start 95.564 109.414) (end 95.564 101.032) (width 0.5) (layer "B.Cu") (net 12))
 (segment (start 72.39 112.776) (end 80.01 120.396) (width 0.5) (layer "B.Cu") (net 12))
 (segment (start 89.224235 115.753765) (end 95.564 109.414) (width 0.5) (layer "B.Cu") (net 12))
 (segment (start 100.28 99) (end 102.5 96.78) (width 0.5) (layer "B.Cu") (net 12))
 (segment (start 97.402 99) (end 100.28 99) (width 0.5) (layer "B.Cu") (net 12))
 (segment (start 87.651434 120.396) (end 89.224235 118.823199) (width 0.5) (layer "B.Cu") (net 12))
 (segment (start 71.882 83.312) (end 66.548 88.646) (width 0.5) (layer "B.Cu") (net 12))
 (segment (start 80.01 120.396) (end 87.651434 120.396) (width 0.5) (layer "B.Cu") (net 12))
 (segment (start 66.548 88.646) (end 66.548 96.774) (width 0.5) (layer "B.Cu") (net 12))
 (segment (start 89.224235 118.823199) (end 89.224235 115.753765) (width 0.5) (layer "B.Cu") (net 12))
 (segment (start 72.39 99.39) (end 72.39 112.776) (width 0.5) (layer "B.Cu") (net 12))
 (segment (start 93.726 99) (end 95.564 100.838) (width 0.5) (layer "B.Cu") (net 12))
 (segment (start 121.168 121.92) (end 122.946 120.142) (width 0.5) (layer "B.Cu") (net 4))
 (segment (start 135.568 120.142) (end 137.6 122.174) (width 0.5) (layer "B.Cu") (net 4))
 (segment (start 122.946 120.142) (end 135.568 120.142) (width 0.5) (layer "B.Cu") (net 4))
 (segment (start 140.14 122.174) (end 137.408 119.442) (width 0.5) (layer "B.Cu") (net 3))
 (segment (start 121.106 119.442) (end 118.628 121.92) (width 0.5) (layer "B.Cu") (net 3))
 (segment (start 137.408 119.442) (end 121.106 119.442) (width 0.5) (layer "B.Cu") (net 3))
 (segment (start 168.651 107.955) (end 157.92 118.686) (width 0.5) (layer "B.Cu") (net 28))
 (segment (start 168.651 106.68) (end 168.651 107.955) (width 0.5) (layer "B.Cu") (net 28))
 (segment (start 157.92 118.686) (end 157.92 122.174) (width 0.5) (layer "B.Cu") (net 28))
 (segment (start 160.46 118.178) (end 160.46 122.174) (width 0.5) (layer "B.Cu") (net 27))
 (segment (start 171.191 107.447) (end 160.46 118.178) (width 0.5) (layer "B.Cu") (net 27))
 (segment (start 171.191 106.68) (end 171.191 107.447) (width 0.5) (layer "B.Cu") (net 27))
 (segment (start 84.221412 99.868588) (end 90.17 93.92) (width 0.5) (layer "B.Cu") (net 6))
 (segment (start 90.17 93.92) (end 69 93.92) (width 0.5) (layer "B.Cu") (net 6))
 (segment (start 96.26 87.83) (end 96.26 81.54) (width 0.5) (layer "B.Cu") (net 6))
 (segment (start 84.221412 117.941066) (end 84.221412 99.868588) (width 0.5) (layer "B.Cu") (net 6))
 (segment (start 96.26 80.476386) (end 94.22468 78.441066) (width 0.5) (layer "B.Cu") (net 6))
 (segment (start 102.5 81.54) (end 96.26 81.54) (width 0.5) (layer "B.Cu") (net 6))
 (segment (start 96.26 81.54) (end 96.26 80.476386) (width 0.5) (layer "B.Cu") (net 6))
 (segment (start 90.17 93.92) (end 96.26 87.83) (width 0.5) (layer "B.Cu") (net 6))
 (segment (start 166.116 108.712) (end 166.116 101.346) (width 0.5) (layer "B.Cu") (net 18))
 (segment (start 136.574 97.79) (end 127.44 106.924) (width 0.5) (layer "B.Cu") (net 18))
 (segment (start 102.5 114.56) (end 106.558 118.618) (width 0.5) (layer "B.Cu") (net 18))
 (segment (start 166.116 101.346) (end 162.56 97.79) (width 0.5) (layer "B.Cu") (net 18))
 (segment (start 106.558 118.618) (end 156.21 118.618) (width 0.5) (layer "B.Cu") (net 18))
 (segment (start 166.116 101.346) (end 172.962 94.5) (width 0.5) (layer "B.Cu") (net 18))
 (segment (start 156.21 118.618) (end 166.116 108.712) (width 0.5) (layer "B.Cu") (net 18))
 (segment (start 162.56 97.79) (end 136.574 97.79) (width 0.5) (layer "B.Cu") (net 18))
 (segment (start 172.962 94.5) (end 185 94.5) (width 0.5) (layer "B.Cu") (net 18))
 (segment (start 175.26 105.156) (end 175.26 106.934) (width 0.5) (layer "B.Cu") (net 25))
 (segment (start 189.992 84.089) (end 188.707 84.089) (width 0.5) (layer "B.Cu") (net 25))
 (segment (start 187.452 85.344) (end 187.452 97.79) (width 0.5) (layer "B.Cu") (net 25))
 (segment (start 187.452 97.79) (end 182.626 97.79) (width 0.5) (layer "B.Cu") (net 25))
 (segment (start 188.707 84.089) (end 187.452 85.344) (width 0.5) (layer "B.Cu") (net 25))
 (segment (start 182.626 97.79) (end 175.26 105.156) (width 0.5) (layer "B.Cu") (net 25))
 (segment (start 114.046 103.024) (end 117.75 99.32) (width 0.5) (layer "B.Cu") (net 35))
 (segment (start 144.51 117.794) (end 155.38 106.924) (width 0.5) (layer "B.Cu") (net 35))
 (segment (start 114.046 117.794) (end 114.046 103.024) (width 0.5) (layer "B.Cu") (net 35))
 (segment (start 144.51 117.794) (end 114.046 117.794) (width 0.5) (layer "B.Cu") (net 35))
 (segment (start 117.75 101.86) (end 114.808 104.802) (width 0.5) (layer "B.Cu") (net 36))
 (segment (start 142.67 117.094) (end 152.84 106.924) (width 0.5) (layer "B.Cu") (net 36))
 (segment (start 115.062 117.094) (end 142.67 117.094) (width 0.5) (layer "B.Cu") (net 36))
 (segment (start 114.808 116.84) (end 115.062 117.094) (width 0.5) (layer "B.Cu") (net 36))
 (segment (start 114.808 104.802) (end 114.808 116.84) (width 0.5) (layer "B.Cu") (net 36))
 (segment (start 129.62 116.394) (end 115.57 116.394) (width 0.5) (layer "B.Cu") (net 37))
 (segment (start 140.892 116.332) (end 150.3 106.924) (width 0.5) (layer "B.Cu") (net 37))
 (segment (start 140.892 116.332) (end 129.682 116.332) (width 0.5) (layer "B.Cu") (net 37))
 (segment (start 115.57 106.58) (end 117.75 104.4) (width 0.5) (layer "B.Cu") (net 37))
 (segment (start 129.682 116.332) (end 129.62 116.394) (width 0.5) (layer "B.Cu") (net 37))
 (segment (start 115.57 116.394) (end 115.57 106.58) (width 0.5) (layer "B.Cu") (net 37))
 (segment (start 113.548 121.92) (end 104.653 121.92) (width 0.5) (layer "B.Cu") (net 1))
 (segment (start 104.653 121.92) (end 104.648 121.925) (width 0.5) (layer "B.Cu") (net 1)))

